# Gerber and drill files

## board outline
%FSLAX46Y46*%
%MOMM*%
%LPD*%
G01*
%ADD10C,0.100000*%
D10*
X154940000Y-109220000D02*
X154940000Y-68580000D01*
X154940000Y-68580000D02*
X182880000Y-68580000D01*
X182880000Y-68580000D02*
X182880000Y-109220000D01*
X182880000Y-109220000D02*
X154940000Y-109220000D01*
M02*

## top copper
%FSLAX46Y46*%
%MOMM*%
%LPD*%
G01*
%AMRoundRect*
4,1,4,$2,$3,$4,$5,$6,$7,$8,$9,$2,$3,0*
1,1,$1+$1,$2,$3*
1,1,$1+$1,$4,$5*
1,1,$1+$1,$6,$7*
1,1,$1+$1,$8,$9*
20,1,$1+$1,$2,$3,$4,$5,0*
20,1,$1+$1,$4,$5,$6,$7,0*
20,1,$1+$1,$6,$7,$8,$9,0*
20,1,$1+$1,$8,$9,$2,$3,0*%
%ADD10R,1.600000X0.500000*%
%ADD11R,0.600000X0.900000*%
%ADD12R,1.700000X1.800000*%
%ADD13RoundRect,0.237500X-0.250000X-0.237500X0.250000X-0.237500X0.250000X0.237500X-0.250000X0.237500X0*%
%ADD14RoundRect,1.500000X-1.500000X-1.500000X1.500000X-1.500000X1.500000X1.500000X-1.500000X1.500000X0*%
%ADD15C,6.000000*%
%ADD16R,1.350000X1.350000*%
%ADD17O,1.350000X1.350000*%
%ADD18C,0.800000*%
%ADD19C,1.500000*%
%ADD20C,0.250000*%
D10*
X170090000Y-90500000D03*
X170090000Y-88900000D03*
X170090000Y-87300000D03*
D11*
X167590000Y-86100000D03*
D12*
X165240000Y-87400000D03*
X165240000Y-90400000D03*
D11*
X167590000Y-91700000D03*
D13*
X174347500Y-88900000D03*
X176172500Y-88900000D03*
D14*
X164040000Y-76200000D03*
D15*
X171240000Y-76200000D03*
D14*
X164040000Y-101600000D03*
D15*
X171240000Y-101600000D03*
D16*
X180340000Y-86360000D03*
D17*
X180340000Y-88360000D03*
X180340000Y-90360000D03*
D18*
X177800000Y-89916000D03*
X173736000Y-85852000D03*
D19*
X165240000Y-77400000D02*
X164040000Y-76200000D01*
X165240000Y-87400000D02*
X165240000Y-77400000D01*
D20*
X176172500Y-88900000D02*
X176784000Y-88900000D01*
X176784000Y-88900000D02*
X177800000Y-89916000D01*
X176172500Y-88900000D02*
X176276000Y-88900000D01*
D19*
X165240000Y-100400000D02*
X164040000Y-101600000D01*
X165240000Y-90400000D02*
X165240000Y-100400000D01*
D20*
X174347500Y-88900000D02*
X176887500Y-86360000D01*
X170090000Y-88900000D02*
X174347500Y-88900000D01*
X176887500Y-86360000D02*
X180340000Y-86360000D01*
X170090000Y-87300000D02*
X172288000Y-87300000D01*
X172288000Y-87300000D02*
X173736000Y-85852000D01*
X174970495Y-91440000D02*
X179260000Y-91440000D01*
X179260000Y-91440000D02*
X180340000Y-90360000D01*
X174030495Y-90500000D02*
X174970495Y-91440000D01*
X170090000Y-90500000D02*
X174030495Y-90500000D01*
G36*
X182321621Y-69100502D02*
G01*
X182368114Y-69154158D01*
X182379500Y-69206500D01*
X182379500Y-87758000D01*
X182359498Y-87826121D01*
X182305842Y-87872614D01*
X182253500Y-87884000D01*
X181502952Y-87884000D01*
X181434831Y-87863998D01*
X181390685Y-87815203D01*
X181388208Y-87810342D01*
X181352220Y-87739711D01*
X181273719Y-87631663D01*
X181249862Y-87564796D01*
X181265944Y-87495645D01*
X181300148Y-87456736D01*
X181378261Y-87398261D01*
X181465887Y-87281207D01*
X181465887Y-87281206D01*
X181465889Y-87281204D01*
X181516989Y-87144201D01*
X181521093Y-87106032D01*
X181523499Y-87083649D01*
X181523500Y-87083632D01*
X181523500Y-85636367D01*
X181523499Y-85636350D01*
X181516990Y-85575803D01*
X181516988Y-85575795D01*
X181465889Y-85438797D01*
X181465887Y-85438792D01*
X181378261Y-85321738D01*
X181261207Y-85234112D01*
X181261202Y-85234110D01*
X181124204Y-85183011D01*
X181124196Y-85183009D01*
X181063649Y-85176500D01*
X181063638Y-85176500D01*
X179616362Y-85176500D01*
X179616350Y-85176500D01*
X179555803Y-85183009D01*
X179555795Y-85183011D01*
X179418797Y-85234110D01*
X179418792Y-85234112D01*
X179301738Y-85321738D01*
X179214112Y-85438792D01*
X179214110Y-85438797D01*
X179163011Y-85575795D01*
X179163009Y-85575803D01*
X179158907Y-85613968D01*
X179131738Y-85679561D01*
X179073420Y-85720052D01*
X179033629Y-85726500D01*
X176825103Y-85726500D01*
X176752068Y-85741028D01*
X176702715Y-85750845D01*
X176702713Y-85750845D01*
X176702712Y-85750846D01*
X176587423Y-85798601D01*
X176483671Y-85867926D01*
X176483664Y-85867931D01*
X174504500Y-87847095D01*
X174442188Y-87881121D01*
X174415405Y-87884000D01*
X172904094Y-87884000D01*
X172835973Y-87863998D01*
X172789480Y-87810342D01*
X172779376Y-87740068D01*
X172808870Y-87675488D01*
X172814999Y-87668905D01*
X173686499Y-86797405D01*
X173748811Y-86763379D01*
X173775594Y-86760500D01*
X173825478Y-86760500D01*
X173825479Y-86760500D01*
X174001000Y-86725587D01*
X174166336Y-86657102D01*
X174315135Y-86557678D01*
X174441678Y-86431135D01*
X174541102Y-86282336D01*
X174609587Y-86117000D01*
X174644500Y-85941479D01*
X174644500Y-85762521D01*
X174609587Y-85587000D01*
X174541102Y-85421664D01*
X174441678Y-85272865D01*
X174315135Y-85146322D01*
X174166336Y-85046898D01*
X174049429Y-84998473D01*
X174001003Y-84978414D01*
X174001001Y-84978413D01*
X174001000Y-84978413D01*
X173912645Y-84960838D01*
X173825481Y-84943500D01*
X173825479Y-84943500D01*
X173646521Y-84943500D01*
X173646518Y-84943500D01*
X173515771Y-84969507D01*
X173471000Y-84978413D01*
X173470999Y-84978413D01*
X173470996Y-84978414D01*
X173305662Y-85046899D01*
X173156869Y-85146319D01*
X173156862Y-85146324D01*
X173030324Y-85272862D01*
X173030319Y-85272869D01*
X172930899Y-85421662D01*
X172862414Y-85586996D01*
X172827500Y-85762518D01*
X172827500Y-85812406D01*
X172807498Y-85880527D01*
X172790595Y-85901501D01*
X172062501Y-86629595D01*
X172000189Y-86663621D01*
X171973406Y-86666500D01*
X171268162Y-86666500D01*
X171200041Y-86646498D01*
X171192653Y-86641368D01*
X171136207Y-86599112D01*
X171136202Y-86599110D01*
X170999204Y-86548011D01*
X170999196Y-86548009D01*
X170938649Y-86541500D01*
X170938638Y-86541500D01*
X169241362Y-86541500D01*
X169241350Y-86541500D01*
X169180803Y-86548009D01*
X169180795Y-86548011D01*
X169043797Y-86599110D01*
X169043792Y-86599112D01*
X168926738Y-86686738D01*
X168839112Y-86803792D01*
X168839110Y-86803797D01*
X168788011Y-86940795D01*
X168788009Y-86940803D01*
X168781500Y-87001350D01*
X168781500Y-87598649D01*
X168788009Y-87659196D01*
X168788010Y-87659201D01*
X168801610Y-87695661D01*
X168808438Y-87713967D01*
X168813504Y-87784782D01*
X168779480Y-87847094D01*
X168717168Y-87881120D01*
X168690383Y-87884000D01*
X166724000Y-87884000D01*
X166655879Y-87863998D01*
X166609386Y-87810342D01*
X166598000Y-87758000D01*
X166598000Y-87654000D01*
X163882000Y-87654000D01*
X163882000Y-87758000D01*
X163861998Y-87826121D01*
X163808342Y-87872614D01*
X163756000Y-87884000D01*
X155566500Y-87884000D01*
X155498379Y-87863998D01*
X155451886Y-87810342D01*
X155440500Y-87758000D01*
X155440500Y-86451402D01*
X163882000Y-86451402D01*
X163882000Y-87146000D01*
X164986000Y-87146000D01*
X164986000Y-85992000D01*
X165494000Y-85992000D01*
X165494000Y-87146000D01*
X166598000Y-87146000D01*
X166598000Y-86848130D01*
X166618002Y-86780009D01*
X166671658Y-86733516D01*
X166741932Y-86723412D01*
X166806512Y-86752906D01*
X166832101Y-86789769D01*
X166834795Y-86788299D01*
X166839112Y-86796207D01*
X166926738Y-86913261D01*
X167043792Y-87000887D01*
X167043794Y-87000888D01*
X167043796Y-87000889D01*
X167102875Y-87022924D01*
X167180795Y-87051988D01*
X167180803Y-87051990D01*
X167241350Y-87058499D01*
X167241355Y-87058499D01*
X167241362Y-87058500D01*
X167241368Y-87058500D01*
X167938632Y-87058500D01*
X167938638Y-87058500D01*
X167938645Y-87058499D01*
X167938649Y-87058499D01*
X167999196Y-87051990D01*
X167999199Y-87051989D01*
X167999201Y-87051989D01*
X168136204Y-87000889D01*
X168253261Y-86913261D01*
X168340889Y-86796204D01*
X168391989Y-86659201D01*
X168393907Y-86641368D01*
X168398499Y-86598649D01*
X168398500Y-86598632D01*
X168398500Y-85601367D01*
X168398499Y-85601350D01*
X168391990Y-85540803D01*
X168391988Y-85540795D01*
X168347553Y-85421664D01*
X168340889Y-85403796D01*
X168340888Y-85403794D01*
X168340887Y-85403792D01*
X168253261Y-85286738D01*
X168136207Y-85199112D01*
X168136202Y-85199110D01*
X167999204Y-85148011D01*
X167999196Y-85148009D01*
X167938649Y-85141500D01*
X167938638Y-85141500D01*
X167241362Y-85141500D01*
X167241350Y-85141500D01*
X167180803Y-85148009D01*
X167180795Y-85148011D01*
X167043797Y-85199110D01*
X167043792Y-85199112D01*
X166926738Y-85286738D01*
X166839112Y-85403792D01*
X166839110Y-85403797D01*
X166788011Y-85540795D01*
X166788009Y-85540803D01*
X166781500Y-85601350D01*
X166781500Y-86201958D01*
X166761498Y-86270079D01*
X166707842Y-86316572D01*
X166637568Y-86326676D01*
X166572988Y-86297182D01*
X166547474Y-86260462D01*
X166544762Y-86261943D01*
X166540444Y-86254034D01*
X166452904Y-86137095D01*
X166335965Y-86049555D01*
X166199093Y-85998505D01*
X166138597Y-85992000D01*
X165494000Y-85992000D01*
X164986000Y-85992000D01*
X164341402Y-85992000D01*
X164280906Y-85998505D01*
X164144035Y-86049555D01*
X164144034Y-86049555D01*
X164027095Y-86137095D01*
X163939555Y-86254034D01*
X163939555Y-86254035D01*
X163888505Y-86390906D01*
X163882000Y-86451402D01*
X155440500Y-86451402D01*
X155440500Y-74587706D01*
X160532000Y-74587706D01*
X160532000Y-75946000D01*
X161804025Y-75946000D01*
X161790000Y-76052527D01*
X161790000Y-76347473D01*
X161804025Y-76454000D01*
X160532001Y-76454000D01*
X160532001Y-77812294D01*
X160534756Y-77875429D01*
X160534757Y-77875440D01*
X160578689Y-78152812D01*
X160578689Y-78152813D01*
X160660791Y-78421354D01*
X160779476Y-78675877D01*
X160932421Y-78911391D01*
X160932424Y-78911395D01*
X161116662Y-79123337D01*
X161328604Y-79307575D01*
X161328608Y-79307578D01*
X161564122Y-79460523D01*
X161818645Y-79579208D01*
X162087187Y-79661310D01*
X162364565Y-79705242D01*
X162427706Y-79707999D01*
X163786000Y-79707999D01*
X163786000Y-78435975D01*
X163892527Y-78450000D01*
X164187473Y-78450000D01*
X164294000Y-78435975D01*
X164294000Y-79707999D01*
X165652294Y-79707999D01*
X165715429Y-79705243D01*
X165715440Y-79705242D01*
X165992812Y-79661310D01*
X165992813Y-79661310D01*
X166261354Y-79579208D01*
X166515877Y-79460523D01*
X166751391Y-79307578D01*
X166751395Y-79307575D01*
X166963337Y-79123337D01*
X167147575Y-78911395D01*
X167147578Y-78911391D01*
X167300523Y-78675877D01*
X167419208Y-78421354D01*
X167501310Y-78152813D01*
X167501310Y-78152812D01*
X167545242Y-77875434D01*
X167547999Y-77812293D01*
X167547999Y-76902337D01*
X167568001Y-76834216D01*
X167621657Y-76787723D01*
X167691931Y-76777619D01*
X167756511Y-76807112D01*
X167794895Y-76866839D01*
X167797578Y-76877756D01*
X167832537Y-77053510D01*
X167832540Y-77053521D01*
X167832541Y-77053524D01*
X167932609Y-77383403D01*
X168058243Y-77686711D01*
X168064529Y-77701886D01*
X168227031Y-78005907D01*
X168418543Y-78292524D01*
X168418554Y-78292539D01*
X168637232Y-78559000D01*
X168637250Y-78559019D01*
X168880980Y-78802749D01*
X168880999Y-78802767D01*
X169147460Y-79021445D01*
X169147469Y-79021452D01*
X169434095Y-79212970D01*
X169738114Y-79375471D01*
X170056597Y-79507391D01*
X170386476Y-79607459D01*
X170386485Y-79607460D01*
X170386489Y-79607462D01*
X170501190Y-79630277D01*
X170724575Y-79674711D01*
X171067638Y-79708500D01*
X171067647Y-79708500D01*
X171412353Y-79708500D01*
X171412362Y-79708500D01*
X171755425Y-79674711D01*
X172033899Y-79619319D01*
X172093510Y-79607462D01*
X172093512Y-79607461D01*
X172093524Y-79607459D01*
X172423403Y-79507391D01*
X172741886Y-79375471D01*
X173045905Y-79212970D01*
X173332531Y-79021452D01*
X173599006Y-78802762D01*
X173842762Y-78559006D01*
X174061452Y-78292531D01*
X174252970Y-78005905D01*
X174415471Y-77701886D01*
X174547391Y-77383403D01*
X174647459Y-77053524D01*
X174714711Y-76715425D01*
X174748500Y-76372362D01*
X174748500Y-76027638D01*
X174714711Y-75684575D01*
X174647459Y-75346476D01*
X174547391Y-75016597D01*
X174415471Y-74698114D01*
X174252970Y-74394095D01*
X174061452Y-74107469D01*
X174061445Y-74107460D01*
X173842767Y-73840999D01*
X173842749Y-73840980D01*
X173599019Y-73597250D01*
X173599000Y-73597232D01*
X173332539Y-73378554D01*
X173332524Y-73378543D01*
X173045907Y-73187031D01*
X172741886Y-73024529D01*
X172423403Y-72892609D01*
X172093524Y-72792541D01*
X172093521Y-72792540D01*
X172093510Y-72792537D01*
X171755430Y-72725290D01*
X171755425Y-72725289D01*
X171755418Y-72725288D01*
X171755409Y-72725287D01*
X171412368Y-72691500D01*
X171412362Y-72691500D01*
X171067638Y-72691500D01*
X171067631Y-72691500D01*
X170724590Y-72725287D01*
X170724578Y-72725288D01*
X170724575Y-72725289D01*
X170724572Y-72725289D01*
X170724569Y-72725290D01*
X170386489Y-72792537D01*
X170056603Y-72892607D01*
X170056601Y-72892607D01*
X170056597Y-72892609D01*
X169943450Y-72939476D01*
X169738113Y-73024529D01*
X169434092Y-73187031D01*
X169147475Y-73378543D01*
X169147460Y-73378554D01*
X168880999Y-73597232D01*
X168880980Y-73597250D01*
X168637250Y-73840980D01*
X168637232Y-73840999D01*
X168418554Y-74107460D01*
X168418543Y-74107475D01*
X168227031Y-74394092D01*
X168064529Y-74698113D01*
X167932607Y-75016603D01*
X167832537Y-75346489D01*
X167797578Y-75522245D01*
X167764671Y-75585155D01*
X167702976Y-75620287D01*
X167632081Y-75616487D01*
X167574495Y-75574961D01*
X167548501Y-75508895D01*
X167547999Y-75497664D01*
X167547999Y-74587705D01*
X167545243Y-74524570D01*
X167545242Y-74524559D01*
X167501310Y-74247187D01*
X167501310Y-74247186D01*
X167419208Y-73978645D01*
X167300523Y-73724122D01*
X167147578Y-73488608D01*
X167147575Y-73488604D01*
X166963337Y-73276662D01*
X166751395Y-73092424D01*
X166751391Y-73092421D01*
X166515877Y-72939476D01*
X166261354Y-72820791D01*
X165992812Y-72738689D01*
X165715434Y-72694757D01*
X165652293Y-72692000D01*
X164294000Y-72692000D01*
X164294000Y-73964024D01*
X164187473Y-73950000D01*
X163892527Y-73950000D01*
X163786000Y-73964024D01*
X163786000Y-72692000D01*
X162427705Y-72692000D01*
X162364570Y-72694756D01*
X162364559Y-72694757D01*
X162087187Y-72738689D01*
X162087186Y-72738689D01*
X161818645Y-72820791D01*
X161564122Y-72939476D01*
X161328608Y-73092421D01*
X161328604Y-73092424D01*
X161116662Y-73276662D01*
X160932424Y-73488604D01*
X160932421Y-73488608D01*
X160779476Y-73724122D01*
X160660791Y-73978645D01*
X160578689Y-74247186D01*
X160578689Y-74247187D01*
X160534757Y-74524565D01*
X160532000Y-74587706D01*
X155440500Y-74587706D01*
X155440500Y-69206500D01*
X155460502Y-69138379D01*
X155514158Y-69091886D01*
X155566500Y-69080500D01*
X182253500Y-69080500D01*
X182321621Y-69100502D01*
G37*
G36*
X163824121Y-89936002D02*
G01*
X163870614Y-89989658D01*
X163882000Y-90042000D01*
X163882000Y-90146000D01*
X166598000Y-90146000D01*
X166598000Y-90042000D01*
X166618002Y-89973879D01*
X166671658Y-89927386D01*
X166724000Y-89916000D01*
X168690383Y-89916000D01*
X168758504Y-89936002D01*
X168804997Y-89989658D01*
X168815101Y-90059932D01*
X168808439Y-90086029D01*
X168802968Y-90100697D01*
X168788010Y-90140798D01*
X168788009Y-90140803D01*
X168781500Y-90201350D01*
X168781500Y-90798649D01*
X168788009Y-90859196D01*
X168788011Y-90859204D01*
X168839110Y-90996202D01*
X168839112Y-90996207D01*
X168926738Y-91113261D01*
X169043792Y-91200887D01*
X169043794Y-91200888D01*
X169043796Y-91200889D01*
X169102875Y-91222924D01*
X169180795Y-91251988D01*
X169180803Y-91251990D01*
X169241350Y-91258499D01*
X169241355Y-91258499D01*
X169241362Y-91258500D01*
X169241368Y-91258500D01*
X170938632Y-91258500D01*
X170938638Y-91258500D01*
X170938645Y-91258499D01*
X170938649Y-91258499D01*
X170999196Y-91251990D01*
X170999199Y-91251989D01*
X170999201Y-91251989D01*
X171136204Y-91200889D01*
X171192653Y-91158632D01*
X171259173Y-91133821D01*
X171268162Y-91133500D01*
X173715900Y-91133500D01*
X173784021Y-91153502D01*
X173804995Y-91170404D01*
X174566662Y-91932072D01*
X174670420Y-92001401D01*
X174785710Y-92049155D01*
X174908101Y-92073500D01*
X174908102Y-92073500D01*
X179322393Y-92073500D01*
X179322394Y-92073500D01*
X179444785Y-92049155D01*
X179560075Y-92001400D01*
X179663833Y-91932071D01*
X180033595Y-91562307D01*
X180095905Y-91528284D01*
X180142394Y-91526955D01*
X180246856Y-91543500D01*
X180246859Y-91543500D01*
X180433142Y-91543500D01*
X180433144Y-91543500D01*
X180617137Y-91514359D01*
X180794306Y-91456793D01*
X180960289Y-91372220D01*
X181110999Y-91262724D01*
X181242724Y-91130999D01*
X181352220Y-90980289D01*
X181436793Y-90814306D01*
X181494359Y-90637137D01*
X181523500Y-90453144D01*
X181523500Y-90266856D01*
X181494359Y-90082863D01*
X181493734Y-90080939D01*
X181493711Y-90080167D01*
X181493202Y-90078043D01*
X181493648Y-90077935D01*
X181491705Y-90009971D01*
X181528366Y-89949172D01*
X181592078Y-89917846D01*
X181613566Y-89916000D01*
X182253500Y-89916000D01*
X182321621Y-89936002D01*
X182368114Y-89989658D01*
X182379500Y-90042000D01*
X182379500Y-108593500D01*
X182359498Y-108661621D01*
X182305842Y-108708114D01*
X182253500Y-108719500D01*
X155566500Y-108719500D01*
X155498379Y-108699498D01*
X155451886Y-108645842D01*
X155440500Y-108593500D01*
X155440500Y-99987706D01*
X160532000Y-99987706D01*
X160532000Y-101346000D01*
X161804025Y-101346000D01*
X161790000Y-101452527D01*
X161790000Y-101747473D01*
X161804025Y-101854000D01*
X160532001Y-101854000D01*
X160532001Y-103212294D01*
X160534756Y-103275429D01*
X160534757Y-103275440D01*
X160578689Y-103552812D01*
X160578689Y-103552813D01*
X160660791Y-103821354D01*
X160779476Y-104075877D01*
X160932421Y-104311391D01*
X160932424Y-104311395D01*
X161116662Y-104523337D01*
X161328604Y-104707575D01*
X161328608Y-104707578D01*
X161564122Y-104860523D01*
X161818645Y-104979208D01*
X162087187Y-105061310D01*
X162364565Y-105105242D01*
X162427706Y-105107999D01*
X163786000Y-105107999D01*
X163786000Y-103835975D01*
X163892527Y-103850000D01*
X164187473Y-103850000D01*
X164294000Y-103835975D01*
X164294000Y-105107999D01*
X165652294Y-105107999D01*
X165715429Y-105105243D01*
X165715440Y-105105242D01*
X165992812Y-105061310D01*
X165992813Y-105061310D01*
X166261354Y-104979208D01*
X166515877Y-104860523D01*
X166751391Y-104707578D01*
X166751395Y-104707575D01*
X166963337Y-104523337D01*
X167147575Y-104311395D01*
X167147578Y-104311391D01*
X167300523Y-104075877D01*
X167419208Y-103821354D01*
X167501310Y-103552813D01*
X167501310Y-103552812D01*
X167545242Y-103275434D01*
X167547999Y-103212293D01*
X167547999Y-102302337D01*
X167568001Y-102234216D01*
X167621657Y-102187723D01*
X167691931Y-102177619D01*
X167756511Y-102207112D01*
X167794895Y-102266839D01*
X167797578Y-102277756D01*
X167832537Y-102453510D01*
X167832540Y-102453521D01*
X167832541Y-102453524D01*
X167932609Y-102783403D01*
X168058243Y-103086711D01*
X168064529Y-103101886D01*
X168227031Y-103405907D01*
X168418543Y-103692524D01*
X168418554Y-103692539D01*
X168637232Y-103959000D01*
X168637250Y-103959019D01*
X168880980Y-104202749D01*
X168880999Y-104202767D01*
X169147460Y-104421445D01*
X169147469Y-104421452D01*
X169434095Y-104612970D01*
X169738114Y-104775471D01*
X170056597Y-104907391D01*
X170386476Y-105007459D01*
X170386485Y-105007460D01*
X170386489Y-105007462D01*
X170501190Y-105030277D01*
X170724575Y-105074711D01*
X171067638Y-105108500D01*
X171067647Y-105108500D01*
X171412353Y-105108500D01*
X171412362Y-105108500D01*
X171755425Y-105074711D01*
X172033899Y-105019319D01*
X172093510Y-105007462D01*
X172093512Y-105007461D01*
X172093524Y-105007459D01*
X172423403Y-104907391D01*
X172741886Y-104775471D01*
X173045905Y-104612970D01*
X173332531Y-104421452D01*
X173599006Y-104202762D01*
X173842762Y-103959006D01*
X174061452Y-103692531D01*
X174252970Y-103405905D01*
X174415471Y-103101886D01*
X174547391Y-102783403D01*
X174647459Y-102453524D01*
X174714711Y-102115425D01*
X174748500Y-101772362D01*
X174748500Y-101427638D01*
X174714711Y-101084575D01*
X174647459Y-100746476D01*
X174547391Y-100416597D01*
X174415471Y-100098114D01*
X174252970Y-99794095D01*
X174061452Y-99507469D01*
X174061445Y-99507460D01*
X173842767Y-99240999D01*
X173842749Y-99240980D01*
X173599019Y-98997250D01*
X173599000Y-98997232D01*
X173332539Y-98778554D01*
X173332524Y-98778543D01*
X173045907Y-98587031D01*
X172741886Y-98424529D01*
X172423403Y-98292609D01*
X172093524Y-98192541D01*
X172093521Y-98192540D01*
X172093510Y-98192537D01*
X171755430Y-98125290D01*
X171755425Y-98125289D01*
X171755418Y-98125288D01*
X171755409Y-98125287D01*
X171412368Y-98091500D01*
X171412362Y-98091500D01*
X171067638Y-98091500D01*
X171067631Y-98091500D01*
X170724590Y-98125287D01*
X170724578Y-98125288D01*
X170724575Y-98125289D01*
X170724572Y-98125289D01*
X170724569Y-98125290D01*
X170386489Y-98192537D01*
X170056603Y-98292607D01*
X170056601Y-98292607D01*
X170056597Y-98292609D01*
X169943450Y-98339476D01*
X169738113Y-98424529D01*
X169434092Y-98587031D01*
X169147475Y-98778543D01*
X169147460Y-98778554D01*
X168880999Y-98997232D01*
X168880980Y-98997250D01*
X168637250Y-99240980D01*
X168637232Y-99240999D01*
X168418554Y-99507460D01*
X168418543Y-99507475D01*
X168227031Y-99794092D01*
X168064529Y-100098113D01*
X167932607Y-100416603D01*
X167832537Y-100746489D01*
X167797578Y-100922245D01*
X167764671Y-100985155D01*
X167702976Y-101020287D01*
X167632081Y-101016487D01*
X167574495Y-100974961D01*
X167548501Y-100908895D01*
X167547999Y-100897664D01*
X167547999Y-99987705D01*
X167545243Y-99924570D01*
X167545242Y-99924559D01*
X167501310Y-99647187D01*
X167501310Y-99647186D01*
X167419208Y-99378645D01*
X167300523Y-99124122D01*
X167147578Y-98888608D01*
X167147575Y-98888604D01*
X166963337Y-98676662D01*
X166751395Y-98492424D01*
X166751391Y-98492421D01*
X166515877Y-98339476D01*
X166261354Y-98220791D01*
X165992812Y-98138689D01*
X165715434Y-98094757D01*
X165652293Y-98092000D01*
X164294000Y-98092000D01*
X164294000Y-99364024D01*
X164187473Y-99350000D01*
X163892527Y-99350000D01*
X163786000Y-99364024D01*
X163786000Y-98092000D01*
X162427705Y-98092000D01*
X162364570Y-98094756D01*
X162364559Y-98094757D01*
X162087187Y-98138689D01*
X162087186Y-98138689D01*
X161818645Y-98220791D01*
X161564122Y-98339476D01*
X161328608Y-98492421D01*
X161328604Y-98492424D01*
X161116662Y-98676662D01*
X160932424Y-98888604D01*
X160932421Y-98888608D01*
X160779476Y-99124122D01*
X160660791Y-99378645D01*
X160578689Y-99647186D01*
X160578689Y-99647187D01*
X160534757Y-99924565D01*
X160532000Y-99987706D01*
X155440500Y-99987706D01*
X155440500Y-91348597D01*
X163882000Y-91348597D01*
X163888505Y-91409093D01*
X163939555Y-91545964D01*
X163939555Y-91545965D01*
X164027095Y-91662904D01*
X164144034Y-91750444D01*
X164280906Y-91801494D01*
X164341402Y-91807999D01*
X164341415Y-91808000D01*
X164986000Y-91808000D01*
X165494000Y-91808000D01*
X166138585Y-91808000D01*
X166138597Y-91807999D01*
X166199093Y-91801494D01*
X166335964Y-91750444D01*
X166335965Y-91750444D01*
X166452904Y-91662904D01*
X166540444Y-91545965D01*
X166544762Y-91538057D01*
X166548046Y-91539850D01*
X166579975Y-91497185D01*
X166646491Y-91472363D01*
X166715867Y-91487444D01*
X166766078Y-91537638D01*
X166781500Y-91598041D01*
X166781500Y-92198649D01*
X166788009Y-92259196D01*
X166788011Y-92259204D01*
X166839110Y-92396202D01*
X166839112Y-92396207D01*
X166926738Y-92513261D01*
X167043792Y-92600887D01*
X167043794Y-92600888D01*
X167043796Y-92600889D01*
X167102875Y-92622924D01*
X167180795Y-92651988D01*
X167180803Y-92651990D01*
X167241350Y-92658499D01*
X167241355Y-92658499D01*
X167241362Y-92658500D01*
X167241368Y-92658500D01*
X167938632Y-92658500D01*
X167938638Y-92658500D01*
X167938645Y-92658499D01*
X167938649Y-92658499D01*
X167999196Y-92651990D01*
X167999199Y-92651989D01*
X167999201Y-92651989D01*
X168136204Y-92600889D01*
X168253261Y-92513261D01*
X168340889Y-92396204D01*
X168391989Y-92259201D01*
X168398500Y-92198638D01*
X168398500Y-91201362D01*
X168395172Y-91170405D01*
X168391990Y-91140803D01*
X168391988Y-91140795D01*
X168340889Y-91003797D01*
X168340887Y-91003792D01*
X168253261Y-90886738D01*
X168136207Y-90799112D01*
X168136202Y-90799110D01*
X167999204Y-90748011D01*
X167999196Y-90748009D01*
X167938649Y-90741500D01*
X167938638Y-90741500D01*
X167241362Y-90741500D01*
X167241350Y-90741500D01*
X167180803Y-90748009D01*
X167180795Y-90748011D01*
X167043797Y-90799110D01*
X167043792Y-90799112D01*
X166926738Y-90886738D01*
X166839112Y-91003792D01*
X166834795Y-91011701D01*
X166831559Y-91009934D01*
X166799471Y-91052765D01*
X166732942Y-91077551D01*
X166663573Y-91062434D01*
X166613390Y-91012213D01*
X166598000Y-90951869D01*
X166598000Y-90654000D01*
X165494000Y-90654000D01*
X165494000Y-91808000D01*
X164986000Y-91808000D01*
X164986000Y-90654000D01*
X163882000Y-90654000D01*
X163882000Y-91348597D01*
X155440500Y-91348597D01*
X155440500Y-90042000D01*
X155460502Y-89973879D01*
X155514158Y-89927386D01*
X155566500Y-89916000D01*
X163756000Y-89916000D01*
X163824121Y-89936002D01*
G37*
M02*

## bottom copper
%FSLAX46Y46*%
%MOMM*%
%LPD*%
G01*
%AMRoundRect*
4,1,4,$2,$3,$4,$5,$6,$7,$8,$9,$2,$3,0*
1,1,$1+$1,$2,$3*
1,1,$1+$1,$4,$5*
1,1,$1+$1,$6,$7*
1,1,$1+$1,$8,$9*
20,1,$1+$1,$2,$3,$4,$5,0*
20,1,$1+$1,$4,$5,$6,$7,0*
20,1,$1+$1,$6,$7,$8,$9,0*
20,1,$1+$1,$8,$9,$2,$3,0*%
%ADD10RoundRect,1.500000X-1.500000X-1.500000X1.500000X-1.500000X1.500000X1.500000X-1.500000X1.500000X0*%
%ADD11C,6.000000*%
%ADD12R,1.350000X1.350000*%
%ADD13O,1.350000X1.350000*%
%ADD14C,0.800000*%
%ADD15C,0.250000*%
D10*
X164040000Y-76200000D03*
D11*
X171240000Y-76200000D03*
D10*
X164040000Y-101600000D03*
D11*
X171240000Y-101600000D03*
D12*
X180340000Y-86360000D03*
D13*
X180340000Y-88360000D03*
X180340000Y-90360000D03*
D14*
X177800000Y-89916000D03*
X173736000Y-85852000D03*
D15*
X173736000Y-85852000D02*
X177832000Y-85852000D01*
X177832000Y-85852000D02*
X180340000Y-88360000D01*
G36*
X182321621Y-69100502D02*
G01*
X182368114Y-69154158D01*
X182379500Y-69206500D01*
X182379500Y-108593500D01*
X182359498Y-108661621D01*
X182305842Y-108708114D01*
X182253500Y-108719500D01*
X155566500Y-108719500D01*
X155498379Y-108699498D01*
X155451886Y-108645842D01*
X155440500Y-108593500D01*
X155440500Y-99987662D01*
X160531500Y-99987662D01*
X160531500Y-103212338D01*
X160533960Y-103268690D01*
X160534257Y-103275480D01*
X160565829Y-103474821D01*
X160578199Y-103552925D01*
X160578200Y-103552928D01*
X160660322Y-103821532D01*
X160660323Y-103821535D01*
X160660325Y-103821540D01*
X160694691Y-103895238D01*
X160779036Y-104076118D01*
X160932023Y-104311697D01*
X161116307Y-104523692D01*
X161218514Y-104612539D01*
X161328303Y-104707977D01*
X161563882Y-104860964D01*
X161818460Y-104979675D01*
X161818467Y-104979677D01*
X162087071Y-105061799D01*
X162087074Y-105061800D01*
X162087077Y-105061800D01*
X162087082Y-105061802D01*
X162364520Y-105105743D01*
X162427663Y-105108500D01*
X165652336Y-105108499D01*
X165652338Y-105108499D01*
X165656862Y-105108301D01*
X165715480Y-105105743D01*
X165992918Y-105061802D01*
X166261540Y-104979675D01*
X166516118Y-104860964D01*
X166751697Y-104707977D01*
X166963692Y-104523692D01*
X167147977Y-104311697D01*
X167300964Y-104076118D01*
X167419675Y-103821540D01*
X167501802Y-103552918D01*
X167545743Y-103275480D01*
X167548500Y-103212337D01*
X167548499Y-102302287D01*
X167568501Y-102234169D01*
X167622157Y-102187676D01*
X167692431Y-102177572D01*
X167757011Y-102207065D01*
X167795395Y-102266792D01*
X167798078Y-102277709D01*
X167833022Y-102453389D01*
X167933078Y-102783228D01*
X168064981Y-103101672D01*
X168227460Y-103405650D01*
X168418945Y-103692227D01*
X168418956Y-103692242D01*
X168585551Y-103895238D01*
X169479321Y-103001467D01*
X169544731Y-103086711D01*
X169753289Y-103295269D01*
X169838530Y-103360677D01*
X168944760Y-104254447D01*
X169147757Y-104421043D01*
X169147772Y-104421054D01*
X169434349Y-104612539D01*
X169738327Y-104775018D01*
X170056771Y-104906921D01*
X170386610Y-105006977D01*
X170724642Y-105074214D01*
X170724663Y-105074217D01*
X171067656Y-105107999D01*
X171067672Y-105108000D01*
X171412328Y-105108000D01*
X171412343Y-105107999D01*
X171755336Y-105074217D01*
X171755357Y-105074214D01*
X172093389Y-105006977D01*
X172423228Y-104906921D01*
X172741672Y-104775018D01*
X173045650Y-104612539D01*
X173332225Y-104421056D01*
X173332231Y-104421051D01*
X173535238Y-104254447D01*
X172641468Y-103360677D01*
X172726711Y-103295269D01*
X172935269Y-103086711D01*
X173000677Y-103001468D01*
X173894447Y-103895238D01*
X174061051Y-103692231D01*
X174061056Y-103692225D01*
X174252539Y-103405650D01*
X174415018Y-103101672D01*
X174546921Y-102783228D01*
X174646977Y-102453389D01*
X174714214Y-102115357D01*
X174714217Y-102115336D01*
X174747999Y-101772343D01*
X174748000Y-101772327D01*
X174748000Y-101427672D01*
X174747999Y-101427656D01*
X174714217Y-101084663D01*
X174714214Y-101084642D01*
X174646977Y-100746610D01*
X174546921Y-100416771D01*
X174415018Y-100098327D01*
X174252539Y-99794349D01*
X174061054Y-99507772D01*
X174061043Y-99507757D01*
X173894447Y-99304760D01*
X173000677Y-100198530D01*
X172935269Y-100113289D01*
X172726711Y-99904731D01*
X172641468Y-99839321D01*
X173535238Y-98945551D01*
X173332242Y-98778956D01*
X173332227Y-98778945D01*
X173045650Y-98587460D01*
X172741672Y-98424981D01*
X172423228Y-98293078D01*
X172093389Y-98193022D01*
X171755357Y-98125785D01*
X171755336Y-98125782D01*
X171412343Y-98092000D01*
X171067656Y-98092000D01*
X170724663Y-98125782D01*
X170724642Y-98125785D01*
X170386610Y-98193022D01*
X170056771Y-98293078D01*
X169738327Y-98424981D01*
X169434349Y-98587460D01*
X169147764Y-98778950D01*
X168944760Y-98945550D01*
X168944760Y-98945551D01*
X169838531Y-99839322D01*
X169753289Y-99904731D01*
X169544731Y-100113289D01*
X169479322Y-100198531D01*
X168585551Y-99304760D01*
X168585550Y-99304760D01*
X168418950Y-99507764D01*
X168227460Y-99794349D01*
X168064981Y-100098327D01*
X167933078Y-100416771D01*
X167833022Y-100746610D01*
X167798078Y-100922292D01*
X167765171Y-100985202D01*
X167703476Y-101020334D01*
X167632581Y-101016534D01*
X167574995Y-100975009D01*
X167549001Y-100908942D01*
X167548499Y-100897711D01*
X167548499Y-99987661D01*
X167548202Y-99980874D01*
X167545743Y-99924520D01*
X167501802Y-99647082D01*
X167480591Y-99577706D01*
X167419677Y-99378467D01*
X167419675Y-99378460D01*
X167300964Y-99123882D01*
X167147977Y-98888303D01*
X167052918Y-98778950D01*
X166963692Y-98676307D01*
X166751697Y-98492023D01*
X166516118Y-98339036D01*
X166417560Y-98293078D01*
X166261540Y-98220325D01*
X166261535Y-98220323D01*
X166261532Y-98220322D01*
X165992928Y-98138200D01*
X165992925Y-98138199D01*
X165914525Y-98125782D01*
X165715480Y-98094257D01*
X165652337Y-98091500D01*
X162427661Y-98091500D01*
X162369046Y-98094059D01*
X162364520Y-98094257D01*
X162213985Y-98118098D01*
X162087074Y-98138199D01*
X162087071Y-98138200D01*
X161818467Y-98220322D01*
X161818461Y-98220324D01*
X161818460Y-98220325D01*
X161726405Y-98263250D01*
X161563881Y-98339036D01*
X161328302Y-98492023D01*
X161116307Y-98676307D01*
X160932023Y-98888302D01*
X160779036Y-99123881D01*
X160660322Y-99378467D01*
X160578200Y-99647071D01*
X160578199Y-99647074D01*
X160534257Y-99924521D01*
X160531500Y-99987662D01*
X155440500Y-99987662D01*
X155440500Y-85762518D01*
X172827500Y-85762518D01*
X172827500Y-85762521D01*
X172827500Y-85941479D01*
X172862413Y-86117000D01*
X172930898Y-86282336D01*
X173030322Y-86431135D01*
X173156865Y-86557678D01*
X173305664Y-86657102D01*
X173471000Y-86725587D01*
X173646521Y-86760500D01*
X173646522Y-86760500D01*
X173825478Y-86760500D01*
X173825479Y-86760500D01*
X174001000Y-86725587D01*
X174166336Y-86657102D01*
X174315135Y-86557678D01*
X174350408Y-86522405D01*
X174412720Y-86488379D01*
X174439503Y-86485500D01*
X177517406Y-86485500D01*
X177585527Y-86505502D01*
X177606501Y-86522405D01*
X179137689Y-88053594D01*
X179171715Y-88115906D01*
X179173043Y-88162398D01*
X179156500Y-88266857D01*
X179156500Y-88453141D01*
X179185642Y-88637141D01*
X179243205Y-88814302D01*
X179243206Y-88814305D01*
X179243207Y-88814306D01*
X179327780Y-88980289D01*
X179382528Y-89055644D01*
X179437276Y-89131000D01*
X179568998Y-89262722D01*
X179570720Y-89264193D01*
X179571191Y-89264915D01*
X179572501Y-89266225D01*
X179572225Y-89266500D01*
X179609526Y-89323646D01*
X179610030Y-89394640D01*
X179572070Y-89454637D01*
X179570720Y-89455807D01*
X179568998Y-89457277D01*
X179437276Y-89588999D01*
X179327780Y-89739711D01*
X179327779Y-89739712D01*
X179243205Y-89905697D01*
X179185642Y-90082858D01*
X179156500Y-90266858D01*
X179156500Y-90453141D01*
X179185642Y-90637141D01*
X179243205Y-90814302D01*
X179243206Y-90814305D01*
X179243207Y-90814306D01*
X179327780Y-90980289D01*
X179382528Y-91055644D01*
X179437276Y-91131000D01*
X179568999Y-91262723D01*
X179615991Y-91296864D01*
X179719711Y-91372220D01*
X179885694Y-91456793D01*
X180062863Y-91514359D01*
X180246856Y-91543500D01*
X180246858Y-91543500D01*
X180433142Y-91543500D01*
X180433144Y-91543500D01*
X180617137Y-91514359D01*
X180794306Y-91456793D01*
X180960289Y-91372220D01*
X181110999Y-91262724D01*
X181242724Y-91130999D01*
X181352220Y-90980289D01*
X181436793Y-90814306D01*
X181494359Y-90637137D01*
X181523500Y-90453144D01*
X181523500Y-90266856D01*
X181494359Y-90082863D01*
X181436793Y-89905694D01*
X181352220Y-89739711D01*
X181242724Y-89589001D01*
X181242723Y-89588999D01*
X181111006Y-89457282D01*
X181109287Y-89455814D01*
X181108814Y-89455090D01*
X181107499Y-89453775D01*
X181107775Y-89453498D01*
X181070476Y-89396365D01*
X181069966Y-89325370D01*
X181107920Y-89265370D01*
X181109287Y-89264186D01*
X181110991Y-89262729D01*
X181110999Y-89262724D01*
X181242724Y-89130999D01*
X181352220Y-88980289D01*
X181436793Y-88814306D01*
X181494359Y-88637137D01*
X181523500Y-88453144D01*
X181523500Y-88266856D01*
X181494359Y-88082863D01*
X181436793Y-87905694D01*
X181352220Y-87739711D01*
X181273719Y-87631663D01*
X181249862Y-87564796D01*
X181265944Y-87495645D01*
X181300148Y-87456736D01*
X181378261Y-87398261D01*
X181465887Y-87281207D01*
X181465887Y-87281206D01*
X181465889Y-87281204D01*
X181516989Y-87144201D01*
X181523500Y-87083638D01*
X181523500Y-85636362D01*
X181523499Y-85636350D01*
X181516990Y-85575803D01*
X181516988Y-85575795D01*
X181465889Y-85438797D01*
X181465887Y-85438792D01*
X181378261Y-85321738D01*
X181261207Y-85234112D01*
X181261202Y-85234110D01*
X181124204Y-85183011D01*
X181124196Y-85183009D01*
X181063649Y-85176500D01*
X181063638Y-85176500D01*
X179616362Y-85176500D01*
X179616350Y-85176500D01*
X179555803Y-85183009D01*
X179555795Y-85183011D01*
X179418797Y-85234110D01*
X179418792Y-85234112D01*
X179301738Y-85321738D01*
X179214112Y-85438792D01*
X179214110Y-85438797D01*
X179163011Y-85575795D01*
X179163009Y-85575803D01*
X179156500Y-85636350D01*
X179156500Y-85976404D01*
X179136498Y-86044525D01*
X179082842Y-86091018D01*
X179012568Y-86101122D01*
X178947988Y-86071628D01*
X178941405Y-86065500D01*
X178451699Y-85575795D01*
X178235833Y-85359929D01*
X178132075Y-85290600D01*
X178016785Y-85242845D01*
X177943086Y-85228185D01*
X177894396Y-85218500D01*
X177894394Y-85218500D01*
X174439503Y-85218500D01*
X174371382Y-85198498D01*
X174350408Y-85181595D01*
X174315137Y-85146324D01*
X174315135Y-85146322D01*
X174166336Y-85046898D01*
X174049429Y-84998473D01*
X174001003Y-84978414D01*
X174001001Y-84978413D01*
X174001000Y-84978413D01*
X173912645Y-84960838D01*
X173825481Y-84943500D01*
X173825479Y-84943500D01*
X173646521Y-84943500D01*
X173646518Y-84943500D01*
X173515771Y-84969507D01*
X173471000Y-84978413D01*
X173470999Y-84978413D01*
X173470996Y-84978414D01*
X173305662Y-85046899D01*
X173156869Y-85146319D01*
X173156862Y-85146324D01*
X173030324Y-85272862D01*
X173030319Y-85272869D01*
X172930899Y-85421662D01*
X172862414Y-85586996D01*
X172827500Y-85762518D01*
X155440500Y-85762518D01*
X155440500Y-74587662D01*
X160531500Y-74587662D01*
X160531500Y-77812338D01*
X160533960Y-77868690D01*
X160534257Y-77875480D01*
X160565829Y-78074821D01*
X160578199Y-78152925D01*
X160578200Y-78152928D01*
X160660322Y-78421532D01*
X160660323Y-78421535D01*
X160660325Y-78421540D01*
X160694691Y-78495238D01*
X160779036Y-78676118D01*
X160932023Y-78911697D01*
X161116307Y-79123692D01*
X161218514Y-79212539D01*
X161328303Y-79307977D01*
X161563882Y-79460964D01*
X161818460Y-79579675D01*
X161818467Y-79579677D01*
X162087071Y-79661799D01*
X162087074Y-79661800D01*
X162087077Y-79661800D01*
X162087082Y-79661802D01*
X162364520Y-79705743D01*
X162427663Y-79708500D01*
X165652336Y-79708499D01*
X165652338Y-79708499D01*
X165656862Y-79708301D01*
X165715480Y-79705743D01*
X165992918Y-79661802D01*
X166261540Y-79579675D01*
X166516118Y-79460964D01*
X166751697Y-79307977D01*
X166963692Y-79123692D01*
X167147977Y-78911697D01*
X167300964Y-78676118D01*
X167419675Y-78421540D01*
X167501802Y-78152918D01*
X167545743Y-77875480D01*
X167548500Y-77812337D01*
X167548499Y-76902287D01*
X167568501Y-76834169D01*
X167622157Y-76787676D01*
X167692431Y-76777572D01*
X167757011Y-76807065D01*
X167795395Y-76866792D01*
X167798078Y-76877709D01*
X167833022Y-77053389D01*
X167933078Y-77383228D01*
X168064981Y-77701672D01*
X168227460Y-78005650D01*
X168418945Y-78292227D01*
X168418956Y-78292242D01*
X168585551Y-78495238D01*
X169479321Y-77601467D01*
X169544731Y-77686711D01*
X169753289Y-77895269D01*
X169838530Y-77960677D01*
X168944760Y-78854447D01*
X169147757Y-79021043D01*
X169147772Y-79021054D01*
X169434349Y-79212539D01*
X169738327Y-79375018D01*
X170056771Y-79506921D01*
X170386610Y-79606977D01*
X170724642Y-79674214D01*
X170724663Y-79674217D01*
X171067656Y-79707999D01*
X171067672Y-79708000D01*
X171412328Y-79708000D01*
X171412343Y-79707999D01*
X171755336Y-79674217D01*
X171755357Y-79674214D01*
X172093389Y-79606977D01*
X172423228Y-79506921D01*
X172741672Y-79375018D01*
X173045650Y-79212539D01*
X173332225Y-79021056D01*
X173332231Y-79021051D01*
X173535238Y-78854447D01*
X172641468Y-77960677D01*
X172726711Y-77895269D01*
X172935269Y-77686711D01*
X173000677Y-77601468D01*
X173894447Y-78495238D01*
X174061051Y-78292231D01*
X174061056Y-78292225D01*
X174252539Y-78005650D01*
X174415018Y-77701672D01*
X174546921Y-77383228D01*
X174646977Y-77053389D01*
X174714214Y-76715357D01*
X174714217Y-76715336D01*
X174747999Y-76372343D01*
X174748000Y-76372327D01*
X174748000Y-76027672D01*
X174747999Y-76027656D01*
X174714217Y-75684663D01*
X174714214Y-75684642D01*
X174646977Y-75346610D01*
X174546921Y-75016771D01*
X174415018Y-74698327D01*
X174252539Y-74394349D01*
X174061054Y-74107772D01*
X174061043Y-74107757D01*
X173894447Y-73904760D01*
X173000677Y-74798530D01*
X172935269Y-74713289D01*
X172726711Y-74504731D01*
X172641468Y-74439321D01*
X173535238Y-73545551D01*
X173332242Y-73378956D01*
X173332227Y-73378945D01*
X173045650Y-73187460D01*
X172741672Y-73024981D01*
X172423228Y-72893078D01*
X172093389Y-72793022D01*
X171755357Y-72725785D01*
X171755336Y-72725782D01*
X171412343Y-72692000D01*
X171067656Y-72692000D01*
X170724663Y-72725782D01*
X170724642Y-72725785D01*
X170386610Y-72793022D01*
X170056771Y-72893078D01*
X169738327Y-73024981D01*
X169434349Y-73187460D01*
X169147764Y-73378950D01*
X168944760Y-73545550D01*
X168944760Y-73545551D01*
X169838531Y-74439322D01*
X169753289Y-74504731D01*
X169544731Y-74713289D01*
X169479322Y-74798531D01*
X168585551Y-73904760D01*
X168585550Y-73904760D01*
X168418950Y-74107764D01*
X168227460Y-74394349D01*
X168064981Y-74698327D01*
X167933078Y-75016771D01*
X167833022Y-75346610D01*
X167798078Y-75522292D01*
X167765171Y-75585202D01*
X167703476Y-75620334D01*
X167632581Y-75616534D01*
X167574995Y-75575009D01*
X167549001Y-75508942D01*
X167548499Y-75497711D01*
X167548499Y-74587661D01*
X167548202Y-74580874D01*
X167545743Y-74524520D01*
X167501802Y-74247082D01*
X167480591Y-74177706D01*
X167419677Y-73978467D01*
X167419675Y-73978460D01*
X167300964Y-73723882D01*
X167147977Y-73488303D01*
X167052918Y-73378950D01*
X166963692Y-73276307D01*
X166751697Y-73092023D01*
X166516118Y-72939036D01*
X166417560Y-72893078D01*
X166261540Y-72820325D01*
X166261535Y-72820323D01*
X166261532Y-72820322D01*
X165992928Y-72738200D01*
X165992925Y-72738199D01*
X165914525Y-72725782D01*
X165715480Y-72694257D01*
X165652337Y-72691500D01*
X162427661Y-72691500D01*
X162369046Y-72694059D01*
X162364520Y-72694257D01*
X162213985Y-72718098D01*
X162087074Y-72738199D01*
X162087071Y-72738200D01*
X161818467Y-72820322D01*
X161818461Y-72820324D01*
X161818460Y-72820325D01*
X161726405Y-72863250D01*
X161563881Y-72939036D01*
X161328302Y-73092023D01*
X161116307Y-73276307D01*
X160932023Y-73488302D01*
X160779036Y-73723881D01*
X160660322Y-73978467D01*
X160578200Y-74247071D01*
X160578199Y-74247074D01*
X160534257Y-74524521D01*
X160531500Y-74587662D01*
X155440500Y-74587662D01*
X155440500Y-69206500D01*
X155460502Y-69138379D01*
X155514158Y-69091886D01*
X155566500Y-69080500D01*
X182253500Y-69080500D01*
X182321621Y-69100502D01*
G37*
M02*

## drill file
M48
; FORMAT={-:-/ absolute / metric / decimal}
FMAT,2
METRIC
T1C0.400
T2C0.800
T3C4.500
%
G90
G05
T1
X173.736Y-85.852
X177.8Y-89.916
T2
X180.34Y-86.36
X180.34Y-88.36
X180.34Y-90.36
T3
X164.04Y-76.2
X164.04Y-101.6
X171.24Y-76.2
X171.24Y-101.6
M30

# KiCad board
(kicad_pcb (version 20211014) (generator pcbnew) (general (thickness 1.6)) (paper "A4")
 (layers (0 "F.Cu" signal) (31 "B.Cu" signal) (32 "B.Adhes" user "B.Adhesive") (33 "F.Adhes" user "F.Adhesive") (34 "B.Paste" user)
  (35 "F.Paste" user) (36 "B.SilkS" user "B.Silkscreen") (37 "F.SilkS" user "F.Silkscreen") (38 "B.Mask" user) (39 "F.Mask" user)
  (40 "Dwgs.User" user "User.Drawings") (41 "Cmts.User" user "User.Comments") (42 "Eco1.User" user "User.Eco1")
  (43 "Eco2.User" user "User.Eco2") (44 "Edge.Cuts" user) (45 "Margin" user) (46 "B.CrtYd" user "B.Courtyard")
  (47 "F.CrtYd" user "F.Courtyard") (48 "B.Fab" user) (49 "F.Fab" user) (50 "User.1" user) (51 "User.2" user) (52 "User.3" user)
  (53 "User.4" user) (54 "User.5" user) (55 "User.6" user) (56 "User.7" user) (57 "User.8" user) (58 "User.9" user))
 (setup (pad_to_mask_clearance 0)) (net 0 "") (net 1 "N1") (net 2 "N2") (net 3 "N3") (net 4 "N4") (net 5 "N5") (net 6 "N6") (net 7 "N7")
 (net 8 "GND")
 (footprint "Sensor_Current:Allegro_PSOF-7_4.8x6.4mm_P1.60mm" (layer "F.Cu") (at 167.64 88.9 180)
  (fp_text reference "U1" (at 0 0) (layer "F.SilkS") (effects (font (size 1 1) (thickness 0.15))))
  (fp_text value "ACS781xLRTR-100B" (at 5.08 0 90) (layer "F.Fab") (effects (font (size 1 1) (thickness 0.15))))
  (pad "1" smd rect (at -2.45 -1.6 180) (size 1.6 0.5) (layers "F.Cu" "F.Paste" "F.Mask") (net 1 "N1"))
  (pad "2" smd rect (at -2.45 0 180) (size 1.6 0.5) (layers "F.Cu" "F.Paste" "F.Mask") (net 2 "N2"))
  (pad "3" smd rect (at -2.45 1.6 180) (size 1.6 0.5) (layers "F.Cu" "F.Paste" "F.Mask") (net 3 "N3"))
  (pad "4" smd rect (at 0.05 2.8 180) (size 0.6 0.9) (layers "F.Cu" "F.Paste" "F.Mask") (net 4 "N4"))
  (pad "5" smd rect (at 2.4 1.5 180) (size 1.7 1.8) (layers "F.Cu" "F.Paste" "F.Mask") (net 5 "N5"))
  (pad "6" smd rect (at 2.4 -1.5 180) (size 1.7 1.8) (layers "F.Cu" "F.Paste" "F.Mask") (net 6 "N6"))
  (pad "7" smd rect (at 0.05 -2.8 180) (size 0.6 0.9) (layers "F.Cu" "F.Paste" "F.Mask") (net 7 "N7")))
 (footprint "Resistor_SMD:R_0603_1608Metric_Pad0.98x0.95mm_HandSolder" (layer "F.Cu") (at 175.26 88.9)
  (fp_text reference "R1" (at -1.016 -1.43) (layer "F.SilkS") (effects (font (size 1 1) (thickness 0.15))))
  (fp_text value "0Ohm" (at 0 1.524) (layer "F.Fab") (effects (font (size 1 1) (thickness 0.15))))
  (pad "1" smd roundrect (at -0.9125 0) (size 0.975 0.95) (layers "F.Cu" "F.Paste" "F.Mask") (roundrect_rratio 0.25) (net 2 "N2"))
  (pad "2" smd roundrect (at 0.9125 0) (size 0.975 0.95) (layers "F.Cu" "F.Paste" "F.Mask") (roundrect_rratio 0.25) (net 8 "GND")))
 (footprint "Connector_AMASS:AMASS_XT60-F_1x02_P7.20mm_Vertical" (layer "F.Cu") (at 164.04 76.2)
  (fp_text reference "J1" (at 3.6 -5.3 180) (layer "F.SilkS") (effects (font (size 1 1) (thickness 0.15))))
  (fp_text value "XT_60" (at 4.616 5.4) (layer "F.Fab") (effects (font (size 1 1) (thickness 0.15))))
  (pad "1" thru_hole roundrect (at 0 0) (size 6 6) (drill 4.5) (layers *.Cu *.Mask) (roundrect_rratio 0.25) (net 5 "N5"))
  (pad "2" thru_hole circle (at 7.2 0) (size 6 6) (drill 4.5) (layers *.Cu *.Mask) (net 8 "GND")))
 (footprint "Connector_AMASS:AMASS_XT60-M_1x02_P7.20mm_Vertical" (layer "F.Cu") (at 164.04 101.6)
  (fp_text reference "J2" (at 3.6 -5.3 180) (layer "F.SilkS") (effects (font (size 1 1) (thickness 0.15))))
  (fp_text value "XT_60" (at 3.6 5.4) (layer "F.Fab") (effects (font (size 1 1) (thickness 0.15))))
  (pad "1" thru_hole roundrect (at 0 0) (size 6 6) (drill 4.5) (layers *.Cu *.Mask) (roundrect_rratio 0.25) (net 6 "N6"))
  (pad "2" thru_hole circle (at 7.2 0) (size 6 6) (drill 4.5) (layers *.Cu *.Mask) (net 8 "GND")))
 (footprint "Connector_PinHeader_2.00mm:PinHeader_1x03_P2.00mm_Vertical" (layer "F.Cu") (at 180.34 86.36)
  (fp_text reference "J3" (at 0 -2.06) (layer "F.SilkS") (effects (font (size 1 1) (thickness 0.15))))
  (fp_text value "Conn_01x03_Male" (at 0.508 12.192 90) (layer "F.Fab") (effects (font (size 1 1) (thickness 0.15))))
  (pad "1" thru_hole rect (at 0 0) (size 1.35 1.35) (drill 0.8) (layers *.Cu *.Mask) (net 2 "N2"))
  (pad "2" thru_hole oval (at 0 2) (size 1.35 1.35) (drill 0.8) (layers *.Cu *.Mask) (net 3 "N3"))
  (pad "3" thru_hole oval (at 0 4) (size 1.35 1.35) (drill 0.8) (layers *.Cu *.Mask) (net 1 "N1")))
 (gr_line (start 154.94 109.22) (end 154.94 68.58) (layer "Edge.Cuts") (width 0.1))
 (gr_line (start 154.94 68.58) (end 182.88 68.58) (layer "Edge.Cuts") (width 0.1))
 (gr_line (start 182.88 68.58) (end 182.88 109.22) (layer "Edge.Cuts") (width 0.1))
 (gr_line (start 182.88 109.22) (end 154.94 109.22) (layer "Edge.Cuts") (width 0.1))
 (segment (start 165.24 77.4) (end 164.04 76.2) (width 1.5) (layer "F.Cu") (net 5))
 (segment (start 165.24 87.4) (end 165.24 77.4) (width 1.5) (layer "F.Cu") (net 5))
 (segment (start 176.1725 88.9) (end 176.784 88.9) (width 0.25) (layer "F.Cu") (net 8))
 (segment (start 176.784 88.9) (end 177.8 89.916) (width 0.25) (layer "F.Cu") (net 8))
 (segment (start 176.1725 88.9) (end 176.276 88.9) (width 0.25) (layer "F.Cu") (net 8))
 (via (at 177.8 89.916) (size 0.8) (drill 0.4) (layers "F.Cu" "B.Cu") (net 8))
 (segment (start 165.24 100.4) (end 164.04 101.6) (width 1.5) (layer "F.Cu") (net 6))
 (segment (start 165.24 90.4) (end 165.24 100.4) (width 1.5) (layer "F.Cu") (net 6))
 (segment (start 174.3475 88.9) (end 176.8875 86.36) (width 0.25) (layer "F.Cu") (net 2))
 (segment (start 170.09 88.9) (end 174.3475 88.9) (width 0.25) (layer "F.Cu") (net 2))
 (segment (start 176.8875 86.36) (end 180.34 86.36) (width 0.25) (layer "F.Cu") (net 2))
 (segment (start 170.09 87.3) (end 172.288 87.3) (width 0.25) (layer "F.Cu") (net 3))
 (segment (start 172.288 87.3) (end 173.736 85.852) (width 0.25) (layer "F.Cu") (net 3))
 (via (at 173.736 85.852) (size 0.8) (drill 0.4) (layers "F.Cu" "B.Cu") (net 3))
 (segment (start 173.736 85.852) (end 177.832 85.852) (width 0.25) (layer "B.Cu") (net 3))
 (segment (start 177.832 85.852) (end 180.34 88.36) (width 0.25) (layer "B.Cu") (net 3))
 (segment (start 174.970495 91.44) (end 179.26 91.44) (width 0.25) (layer "F.Cu") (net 1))
 (segment (start 179.26 91.44) (end 180.34 90.36) (width 0.25) (layer "F.Cu") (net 1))
 (segment (start 174.030495 90.5) (end 174.970495 91.44) (width 0.25) (layer "F.Cu") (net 1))
 (segment (start 170.09 90.5) (end 174.030495 90.5) (width 0.25) (layer "F.Cu") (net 1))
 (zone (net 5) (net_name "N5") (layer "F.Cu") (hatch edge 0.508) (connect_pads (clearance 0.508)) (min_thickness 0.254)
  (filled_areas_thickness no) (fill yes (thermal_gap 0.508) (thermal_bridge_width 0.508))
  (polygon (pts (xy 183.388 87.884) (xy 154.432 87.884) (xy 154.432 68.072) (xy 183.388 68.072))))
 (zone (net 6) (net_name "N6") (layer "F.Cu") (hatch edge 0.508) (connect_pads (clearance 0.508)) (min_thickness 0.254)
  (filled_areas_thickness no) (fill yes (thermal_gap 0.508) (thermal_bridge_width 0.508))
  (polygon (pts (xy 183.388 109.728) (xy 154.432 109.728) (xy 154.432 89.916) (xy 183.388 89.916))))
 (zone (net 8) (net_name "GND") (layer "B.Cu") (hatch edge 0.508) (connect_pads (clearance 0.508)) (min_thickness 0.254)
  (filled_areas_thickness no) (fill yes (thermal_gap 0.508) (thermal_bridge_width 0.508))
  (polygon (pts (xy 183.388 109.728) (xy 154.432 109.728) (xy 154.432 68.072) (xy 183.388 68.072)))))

